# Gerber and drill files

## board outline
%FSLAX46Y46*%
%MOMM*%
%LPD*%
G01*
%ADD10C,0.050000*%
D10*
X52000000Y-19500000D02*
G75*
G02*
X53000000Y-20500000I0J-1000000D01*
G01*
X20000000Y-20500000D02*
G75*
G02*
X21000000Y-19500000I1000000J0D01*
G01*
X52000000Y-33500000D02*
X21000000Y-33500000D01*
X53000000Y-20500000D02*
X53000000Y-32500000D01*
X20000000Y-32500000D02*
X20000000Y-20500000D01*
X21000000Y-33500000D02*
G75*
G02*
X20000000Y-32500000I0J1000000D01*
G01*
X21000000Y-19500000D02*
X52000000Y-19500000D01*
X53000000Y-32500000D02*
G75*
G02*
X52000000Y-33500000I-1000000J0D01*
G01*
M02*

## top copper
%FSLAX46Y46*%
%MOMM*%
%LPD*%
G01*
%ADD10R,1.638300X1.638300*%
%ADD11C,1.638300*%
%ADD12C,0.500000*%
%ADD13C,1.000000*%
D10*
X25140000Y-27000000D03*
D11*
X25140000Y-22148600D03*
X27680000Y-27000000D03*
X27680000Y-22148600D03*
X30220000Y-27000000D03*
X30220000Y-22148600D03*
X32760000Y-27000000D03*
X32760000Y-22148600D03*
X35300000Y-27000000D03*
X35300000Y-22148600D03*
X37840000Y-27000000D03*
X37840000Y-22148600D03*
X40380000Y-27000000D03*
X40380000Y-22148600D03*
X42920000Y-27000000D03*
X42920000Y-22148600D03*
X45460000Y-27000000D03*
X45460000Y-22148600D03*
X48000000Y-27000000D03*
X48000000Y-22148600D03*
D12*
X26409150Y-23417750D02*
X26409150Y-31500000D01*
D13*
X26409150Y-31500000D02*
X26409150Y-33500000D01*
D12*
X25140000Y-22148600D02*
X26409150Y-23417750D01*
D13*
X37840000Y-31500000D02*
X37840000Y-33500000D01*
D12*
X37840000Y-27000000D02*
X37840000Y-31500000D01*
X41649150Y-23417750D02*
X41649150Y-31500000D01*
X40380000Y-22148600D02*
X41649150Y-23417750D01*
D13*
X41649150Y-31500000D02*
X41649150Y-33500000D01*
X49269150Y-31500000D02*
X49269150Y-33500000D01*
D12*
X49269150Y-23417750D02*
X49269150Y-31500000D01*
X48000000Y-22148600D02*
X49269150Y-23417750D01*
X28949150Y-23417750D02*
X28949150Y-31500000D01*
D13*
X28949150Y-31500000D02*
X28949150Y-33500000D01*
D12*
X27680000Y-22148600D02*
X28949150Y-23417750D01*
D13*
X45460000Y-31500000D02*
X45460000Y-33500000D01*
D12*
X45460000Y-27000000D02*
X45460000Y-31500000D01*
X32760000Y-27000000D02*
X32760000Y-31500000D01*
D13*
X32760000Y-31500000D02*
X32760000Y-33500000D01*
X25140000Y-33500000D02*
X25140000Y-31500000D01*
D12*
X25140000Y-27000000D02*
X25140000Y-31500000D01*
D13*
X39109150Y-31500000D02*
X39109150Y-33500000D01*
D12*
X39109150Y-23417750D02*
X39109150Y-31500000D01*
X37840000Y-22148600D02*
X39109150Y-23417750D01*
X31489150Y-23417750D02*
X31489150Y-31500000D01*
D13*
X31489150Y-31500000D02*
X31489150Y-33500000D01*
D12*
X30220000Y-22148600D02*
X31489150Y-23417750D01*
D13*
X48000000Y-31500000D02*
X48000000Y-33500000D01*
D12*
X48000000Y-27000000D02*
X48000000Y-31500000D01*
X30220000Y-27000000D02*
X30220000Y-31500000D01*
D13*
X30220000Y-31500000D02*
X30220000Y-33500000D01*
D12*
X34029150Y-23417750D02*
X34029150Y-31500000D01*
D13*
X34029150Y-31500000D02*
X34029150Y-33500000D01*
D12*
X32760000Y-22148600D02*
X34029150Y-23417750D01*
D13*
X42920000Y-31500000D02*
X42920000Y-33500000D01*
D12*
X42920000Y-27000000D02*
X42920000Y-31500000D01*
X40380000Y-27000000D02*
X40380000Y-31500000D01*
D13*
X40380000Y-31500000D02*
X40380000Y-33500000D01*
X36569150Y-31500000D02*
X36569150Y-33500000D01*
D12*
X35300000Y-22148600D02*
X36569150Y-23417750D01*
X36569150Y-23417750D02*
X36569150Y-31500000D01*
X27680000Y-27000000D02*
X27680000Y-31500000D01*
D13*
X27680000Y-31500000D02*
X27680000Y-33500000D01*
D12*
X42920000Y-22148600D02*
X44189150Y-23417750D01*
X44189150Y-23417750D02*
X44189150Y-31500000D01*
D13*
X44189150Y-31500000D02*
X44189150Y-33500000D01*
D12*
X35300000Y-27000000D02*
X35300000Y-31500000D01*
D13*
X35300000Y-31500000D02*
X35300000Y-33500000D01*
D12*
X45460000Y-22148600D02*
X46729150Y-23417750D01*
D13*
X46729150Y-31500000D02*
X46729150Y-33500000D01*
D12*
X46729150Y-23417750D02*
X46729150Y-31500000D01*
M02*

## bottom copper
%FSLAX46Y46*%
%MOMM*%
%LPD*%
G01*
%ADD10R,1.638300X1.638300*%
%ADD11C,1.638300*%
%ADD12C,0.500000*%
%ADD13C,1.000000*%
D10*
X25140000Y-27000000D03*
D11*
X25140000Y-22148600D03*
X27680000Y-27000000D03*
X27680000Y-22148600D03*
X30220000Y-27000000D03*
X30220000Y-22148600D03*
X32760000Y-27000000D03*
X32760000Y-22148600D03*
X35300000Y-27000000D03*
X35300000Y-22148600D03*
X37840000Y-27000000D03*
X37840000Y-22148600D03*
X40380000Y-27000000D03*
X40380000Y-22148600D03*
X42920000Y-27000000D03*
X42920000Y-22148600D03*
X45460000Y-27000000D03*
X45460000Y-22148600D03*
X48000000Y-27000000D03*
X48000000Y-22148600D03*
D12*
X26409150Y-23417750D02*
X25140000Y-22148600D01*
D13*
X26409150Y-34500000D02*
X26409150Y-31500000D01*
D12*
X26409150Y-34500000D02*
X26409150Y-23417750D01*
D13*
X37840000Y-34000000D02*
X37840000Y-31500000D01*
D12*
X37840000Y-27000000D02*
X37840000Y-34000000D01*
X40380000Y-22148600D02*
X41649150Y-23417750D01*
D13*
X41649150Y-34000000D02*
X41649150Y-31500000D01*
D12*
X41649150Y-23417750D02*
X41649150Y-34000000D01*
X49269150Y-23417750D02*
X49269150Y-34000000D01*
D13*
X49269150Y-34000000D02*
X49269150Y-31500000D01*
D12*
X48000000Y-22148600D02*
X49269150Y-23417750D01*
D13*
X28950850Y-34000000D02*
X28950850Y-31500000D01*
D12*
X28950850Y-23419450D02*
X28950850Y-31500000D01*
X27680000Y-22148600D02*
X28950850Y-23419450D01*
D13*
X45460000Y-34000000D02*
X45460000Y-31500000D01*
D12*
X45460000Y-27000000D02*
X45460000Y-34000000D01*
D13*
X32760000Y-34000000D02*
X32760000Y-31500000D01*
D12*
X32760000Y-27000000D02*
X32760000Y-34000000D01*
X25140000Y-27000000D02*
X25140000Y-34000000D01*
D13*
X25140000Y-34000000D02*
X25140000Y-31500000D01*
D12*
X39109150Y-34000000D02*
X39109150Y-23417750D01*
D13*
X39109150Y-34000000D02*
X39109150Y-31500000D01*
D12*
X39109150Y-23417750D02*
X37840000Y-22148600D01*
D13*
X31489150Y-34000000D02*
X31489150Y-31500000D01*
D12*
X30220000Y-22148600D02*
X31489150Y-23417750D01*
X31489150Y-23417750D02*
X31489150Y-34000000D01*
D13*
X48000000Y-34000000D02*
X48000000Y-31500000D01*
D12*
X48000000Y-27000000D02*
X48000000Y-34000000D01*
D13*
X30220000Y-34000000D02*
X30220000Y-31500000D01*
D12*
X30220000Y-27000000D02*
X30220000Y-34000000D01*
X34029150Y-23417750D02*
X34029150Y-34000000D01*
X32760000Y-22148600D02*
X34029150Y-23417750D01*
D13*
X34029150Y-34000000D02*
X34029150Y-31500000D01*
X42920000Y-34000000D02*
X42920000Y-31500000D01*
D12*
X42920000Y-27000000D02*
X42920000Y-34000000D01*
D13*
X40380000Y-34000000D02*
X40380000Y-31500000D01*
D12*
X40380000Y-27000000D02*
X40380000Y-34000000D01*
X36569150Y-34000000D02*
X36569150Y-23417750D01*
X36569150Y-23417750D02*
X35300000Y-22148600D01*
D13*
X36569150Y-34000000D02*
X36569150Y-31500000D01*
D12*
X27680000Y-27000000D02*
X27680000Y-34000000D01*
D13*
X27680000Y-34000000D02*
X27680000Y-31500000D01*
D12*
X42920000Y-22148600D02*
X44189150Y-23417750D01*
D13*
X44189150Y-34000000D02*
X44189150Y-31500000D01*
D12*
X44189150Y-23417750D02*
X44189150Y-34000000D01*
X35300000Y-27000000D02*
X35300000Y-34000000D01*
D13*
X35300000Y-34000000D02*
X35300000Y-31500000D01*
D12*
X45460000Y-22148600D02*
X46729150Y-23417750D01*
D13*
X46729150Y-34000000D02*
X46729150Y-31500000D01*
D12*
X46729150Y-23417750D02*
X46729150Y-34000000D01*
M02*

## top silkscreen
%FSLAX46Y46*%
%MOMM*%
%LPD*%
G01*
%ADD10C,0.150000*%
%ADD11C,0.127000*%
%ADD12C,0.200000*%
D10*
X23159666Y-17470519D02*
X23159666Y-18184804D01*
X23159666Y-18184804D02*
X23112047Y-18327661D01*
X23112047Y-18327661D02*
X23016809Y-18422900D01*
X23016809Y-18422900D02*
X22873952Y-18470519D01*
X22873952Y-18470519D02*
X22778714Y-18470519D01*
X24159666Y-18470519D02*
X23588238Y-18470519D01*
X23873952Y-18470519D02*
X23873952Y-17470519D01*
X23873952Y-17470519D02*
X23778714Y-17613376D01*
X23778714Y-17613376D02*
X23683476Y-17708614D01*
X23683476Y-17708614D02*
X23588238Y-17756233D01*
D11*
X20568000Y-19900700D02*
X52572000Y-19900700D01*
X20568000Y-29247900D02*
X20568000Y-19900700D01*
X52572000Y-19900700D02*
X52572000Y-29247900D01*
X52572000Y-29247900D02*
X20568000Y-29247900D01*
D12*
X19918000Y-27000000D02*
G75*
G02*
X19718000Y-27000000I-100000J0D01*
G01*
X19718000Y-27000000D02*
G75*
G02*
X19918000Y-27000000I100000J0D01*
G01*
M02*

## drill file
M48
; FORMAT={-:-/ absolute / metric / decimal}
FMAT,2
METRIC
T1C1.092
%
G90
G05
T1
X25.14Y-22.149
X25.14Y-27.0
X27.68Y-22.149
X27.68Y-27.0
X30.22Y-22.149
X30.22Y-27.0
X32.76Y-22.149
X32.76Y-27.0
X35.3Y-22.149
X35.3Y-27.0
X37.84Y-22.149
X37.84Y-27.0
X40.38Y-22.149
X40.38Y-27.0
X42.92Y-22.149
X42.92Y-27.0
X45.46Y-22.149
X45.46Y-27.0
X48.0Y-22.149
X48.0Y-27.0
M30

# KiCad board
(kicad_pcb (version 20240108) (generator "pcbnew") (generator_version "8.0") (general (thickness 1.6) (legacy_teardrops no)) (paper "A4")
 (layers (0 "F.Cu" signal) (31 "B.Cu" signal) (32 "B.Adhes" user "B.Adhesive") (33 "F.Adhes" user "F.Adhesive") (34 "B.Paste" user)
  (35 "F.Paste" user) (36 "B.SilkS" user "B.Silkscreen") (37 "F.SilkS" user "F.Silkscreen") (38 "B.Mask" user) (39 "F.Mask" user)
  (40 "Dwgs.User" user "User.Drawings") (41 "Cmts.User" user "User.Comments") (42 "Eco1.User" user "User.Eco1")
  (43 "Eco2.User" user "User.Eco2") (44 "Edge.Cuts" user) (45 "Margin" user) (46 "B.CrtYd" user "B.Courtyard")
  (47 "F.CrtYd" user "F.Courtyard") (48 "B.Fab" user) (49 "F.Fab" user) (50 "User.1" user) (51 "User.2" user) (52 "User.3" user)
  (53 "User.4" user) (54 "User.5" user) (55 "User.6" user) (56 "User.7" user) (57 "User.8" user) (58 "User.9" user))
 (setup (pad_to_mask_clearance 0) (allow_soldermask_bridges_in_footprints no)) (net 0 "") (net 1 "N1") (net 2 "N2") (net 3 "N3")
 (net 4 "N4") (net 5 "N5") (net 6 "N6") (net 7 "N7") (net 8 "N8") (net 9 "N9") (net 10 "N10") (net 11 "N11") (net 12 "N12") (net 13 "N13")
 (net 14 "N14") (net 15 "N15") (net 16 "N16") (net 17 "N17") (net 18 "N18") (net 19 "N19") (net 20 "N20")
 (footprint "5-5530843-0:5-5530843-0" (layer "F.Cu") (at 36.57 24.5743)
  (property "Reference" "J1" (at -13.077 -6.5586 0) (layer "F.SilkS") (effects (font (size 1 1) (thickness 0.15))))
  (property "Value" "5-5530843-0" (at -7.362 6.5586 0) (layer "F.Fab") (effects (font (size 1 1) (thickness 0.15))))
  (fp_line (start -16.002 -4.6736) (end 16.002 -4.6736) (stroke (width 0.127) (type solid)) (layer "F.SilkS"))
  (fp_line (start -16.002 4.6736) (end -16.002 -4.6736) (stroke (width 0.127) (type solid)) (layer "F.SilkS"))
  (fp_line (start 16.002 -4.6736) (end 16.002 4.6736) (stroke (width 0.127) (type solid)) (layer "F.SilkS"))
  (fp_line (start 16.002 4.6736) (end -16.002 4.6736) (stroke (width 0.127) (type solid)) (layer "F.SilkS"))
  (fp_circle (center -16.752 2.4257) (end -16.652 2.4257) (stroke (width 0.2) (type solid)) (fill none) (layer "F.SilkS"))
  (pad "1" thru_hole rect (at -11.43 2.4257) (size 1.6383 1.6383) (drill 1.0922) (layers "*.Cu" "*.Mask") (remove_unused_layers no)
   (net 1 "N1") (solder_mask_margin 0.102))
  (pad "2" thru_hole circle (at -11.43 -2.4257) (size 1.6383 1.6383) (drill 1.0922) (layers "*.Cu" "*.Mask") (remove_unused_layers no)
   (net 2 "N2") (solder_mask_margin 0.102))
  (pad "3" thru_hole circle (at -8.89 2.4257) (size 1.6383 1.6383) (drill 1.0922) (layers "*.Cu" "*.Mask") (remove_unused_layers no)
   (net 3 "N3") (solder_mask_margin 0.102))
  (pad "4" thru_hole circle (at -8.89 -2.4257) (size 1.6383 1.6383) (drill 1.0922) (layers "*.Cu" "*.Mask") (remove_unused_layers no)
   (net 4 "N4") (solder_mask_margin 0.102))
  (pad "5" thru_hole circle (at -6.35 2.4257) (size 1.6383 1.6383) (drill 1.0922) (layers "*.Cu" "*.Mask") (remove_unused_layers no)
   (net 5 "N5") (solder_mask_margin 0.102))
  (pad "6" thru_hole circle (at -6.35 -2.4257) (size 1.6383 1.6383) (drill 1.0922) (layers "*.Cu" "*.Mask") (remove_unused_layers no)
   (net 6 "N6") (solder_mask_margin 0.102))
  (pad "7" thru_hole circle (at -3.81 2.4257) (size 1.6383 1.6383) (drill 1.0922) (layers "*.Cu" "*.Mask") (remove_unused_layers no)
   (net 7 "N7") (solder_mask_margin 0.102))
  (pad "8" thru_hole circle (at -3.81 -2.4257) (size 1.6383 1.6383) (drill 1.0922) (layers "*.Cu" "*.Mask") (remove_unused_layers no)
   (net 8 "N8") (solder_mask_margin 0.102))
  (pad "9" thru_hole circle (at -1.27 2.4257) (size 1.6383 1.6383) (drill 1.0922) (layers "*.Cu" "*.Mask") (remove_unused_layers no)
   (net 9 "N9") (solder_mask_margin 0.102))
  (pad "10" thru_hole circle (at -1.27 -2.4257) (size 1.6383 1.6383) (drill 1.0922) (layers "*.Cu" "*.Mask") (remove_unused_layers no)
   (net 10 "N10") (solder_mask_margin 0.102))
  (pad "11" thru_hole circle (at 1.27 2.4257) (size 1.6383 1.6383) (drill 1.0922) (layers "*.Cu" "*.Mask") (remove_unused_layers no)
   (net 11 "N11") (solder_mask_margin 0.102))
  (pad "12" thru_hole circle (at 1.27 -2.4257) (size 1.6383 1.6383) (drill 1.0922) (layers "*.Cu" "*.Mask") (remove_unused_layers no)
   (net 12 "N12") (solder_mask_margin 0.102))
  (pad "13" thru_hole circle (at 3.81 2.4257) (size 1.6383 1.6383) (drill 1.0922) (layers "*.Cu" "*.Mask") (remove_unused_layers no)
   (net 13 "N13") (solder_mask_margin 0.102))
  (pad "14" thru_hole circle (at 3.81 -2.4257) (size 1.6383 1.6383) (drill 1.0922) (layers "*.Cu" "*.Mask") (remove_unused_layers no)
   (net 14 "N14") (solder_mask_margin 0.102))
  (pad "15" thru_hole circle (at 6.35 2.4257) (size 1.6383 1.6383) (drill 1.0922) (layers "*.Cu" "*.Mask") (remove_unused_layers no)
   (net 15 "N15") (solder_mask_margin 0.102))
  (pad "16" thru_hole circle (at 6.35 -2.4257) (size 1.6383 1.6383) (drill 1.0922) (layers "*.Cu" "*.Mask") (remove_unused_layers no)
   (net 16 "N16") (solder_mask_margin 0.102))
  (pad "17" thru_hole circle (at 8.89 2.4257) (size 1.6383 1.6383) (drill 1.0922) (layers "*.Cu" "*.Mask") (remove_unused_layers no)
   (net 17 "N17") (solder_mask_margin 0.102))
  (pad "18" thru_hole circle (at 8.89 -2.4257) (size 1.6383 1.6383) (drill 1.0922) (layers "*.Cu" "*.Mask") (remove_unused_layers no)
   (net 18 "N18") (solder_mask_margin 0.102))
  (pad "19" thru_hole circle (at 11.43 2.4257) (size 1.6383 1.6383) (drill 1.0922) (layers "*.Cu" "*.Mask") (remove_unused_layers no)
   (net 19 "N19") (solder_mask_margin 0.102))
  (pad "20" thru_hole circle (at 11.43 -2.4257) (size 1.6383 1.6383) (drill 1.0922) (layers "*.Cu" "*.Mask") (remove_unused_layers no)
   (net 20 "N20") (solder_mask_margin 0.102)))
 (gr_arc (start 52 19.5) (mid 52.707107 19.792893) (end 53 20.5) (stroke (width 0.05) (type default)) (layer "Edge.Cuts"))
 (gr_arc (start 20 20.5) (mid 20.292893 19.792893) (end 21 19.5) (stroke (width 0.05) (type default)) (layer "Edge.Cuts"))
 (gr_line (start 52 33.5) (end 21 33.5) (stroke (width 0.05) (type default)) (layer "Edge.Cuts"))
 (gr_line (start 53 20.5) (end 53 32.5) (stroke (width 0.05) (type default)) (layer "Edge.Cuts"))
 (gr_line (start 20 32.5) (end 20 20.5) (stroke (width 0.05) (type default)) (layer "Edge.Cuts"))
 (gr_arc (start 21 33.5) (mid 20.292893 33.207107) (end 20 32.5) (stroke (width 0.05) (type default)) (layer "Edge.Cuts"))
 (gr_line (start 21 19.5) (end 52 19.5) (stroke (width 0.05) (type default)) (layer "Edge.Cuts"))
 (gr_arc (start 53 32.5) (mid 52.707107 33.207107) (end 52 33.5) (stroke (width 0.05) (type default)) (layer "Edge.Cuts"))
 (segment (start 26.40915 23.41775) (end 26.40915 31.5) (width 0.5) (layer "F.Cu") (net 2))
 (segment (start 26.40915 31.5) (end 26.40915 33.5) (width 1) (layer "F.Cu") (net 2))
 (segment (start 25.14 22.1486) (end 26.40915 23.41775) (width 0.5) (layer "F.Cu") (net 2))
 (segment (start 26.40915 23.41775) (end 25.14 22.1486) (width 0.5) (layer "B.Cu") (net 2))
 (segment (start 26.40915 34.5) (end 26.40915 31.5) (width 1) (layer "B.Cu") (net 2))
 (segment (start 26.40915 34.5) (end 26.40915 23.41775) (width 0.5) (layer "B.Cu") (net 2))
 (segment (start 37.84 31.5) (end 37.84 33.5) (width 1) (layer "F.Cu") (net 11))
 (segment (start 37.84 27) (end 37.84 31.5) (width 0.5) (layer "F.Cu") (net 11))
 (segment (start 37.84 34) (end 37.84 31.5) (width 1) (layer "B.Cu") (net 11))
 (segment (start 37.84 27) (end 37.84 34) (width 0.5) (layer "B.Cu") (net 11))
 (segment (start 41.64915 23.41775) (end 41.64915 31.5) (width 0.5) (layer "F.Cu") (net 14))
 (segment (start 40.38 22.1486) (end 41.64915 23.41775) (width 0.5) (layer "F.Cu") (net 14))
 (segment (start 41.64915 31.5) (end 41.64915 33.5) (width 1) (layer "F.Cu") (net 14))
 (segment (start 40.38 22.1486) (end 41.64915 23.41775) (width 0.5) (layer "B.Cu") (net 14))
 (segment (start 41.64915 34) (end 41.64915 31.5) (width 1) (layer "B.Cu") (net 14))
 (segment (start 41.64915 23.41775) (end 41.64915 34) (width 0.5) (layer "B.Cu") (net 14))
 (segment (start 49.26915 31.5) (end 49.26915 33.5) (width 1) (layer "F.Cu") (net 20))
 (segment (start 49.26915 23.41775) (end 49.26915 31.5) (width 0.5) (layer "F.Cu") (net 20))
 (segment (start 48 22.1486) (end 49.26915 23.41775) (width 0.5) (layer "F.Cu") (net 20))
 (segment (start 49.26915 23.41775) (end 49.26915 34) (width 0.5) (layer "B.Cu") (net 20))
 (segment (start 49.26915 34) (end 49.26915 31.5) (width 1) (layer "B.Cu") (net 20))
 (segment (start 48 22.1486) (end 49.26915 23.41775) (width 0.5) (layer "B.Cu") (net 20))
 (segment (start 28.94915 23.41775) (end 28.94915 31.5) (width 0.5) (layer "F.Cu") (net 4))
 (segment (start 28.94915 31.5) (end 28.94915 33.5) (width 1) (layer "F.Cu") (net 4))
 (segment (start 27.68 22.1486) (end 28.94915 23.41775) (width 0.5) (layer "F.Cu") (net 4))
 (segment (start 28.95085 34) (end 28.95085 31.5) (width 1) (layer "B.Cu") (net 4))
 (segment (start 28.95085 23.41945) (end 28.95085 31.5) (width 0.5) (layer "B.Cu") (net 4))
 (segment (start 27.68 22.1486) (end 28.95085 23.41945) (width 0.5) (layer "B.Cu") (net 4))
 (segment (start 45.46 31.5) (end 45.46 33.5) (width 1) (layer "F.Cu") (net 17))
 (segment (start 45.46 27) (end 45.46 31.5) (width 0.5) (layer "F.Cu") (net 17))
 (segment (start 45.46 34) (end 45.46 31.5) (width 1) (layer "B.Cu") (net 17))
 (segment (start 45.46 27) (end 45.46 34) (width 0.5) (layer "B.Cu") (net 17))
 (segment (start 32.76 27) (end 32.76 31.5) (width 0.5) (layer "F.Cu") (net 7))
 (segment (start 32.76 31.5) (end 32.76 33.5) (width 1) (layer "F.Cu") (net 7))
 (segment (start 32.76 34) (end 32.76 31.5) (width 1) (layer "B.Cu") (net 7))
 (segment (start 32.76 27) (end 32.76 34) (width 0.5) (layer "B.Cu") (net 7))
 (segment (start 25.14 33.5) (end 25.14 31.5) (width 1) (layer "F.Cu") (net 1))
 (segment (start 25.14 27) (end 25.14 31.5) (width 0.5) (layer "F.Cu") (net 1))
 (segment (start 25.14 27) (end 25.14 34) (width 0.5) (layer "B.Cu") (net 1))
 (segment (start 25.14 34) (end 25.14 31.5) (width 1) (layer "B.Cu") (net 1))
 (segment (start 39.10915 31.5) (end 39.10915 33.5) (width 1) (layer "F.Cu") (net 12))
 (segment (start 39.10915 23.41775) (end 39.10915 31.5) (width 0.5) (layer "F.Cu") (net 12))
 (segment (start 37.84 22.1486) (end 39.10915 23.41775) (width 0.5) (layer "F.Cu") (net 12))
 (segment (start 39.10915 34) (end 39.10915 23.41775) (width 0.5) (layer "B.Cu") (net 12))
 (segment (start 39.10915 34) (end 39.10915 31.5) (width 1) (layer "B.Cu") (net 12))
 (segment (start 39.10915 23.41775) (end 37.84 22.1486) (width 0.5) (layer "B.Cu") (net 12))
 (segment (start 31.48915 23.41775) (end 31.48915 31.5) (width 0.5) (layer "F.Cu") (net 6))
 (segment (start 31.48915 31.5) (end 31.48915 33.5) (width 1) (layer "F.Cu") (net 6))
 (segment (start 30.22 22.1486) (end 31.48915 23.41775) (width 0.5) (layer "F.Cu") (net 6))
 (segment (start 31.48915 34) (end 31.48915 31.5) (width 1) (layer "B.Cu") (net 6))
 (segment (start 30.22 22.1486) (end 31.48915 23.41775) (width 0.5) (layer "B.Cu") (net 6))
 (segment (start 31.48915 23.41775) (end 31.48915 34) (width 0.5) (layer "B.Cu") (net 6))
 (segment (start 48 31.5) (end 48 33.5) (width 1) (layer "F.Cu") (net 19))
 (segment (start 48 27) (end 48 31.5) (width 0.5) (layer "F.Cu") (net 19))
 (segment (start 48 34) (end 48 31.5) (width 1) (layer "B.Cu") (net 19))
 (segment (start 48 27) (end 48 34) (width 0.5) (layer "B.Cu") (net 19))
 (segment (start 30.22 27) (end 30.22 31.5) (width 0.5) (layer "F.Cu") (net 5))
 (segment (start 30.22 31.5) (end 30.22 33.5) (width 1) (layer "F.Cu") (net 5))
 (segment (start 30.22 34) (end 30.22 31.5) (width 1) (layer "B.Cu") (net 5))
 (segment (start 30.22 27) (end 30.22 34) (width 0.5) (layer "B.Cu") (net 5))
 (segment (start 34.02915 23.41775) (end 34.02915 31.5) (width 0.5) (layer "F.Cu") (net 8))
 (segment (start 34.02915 31.5) (end 34.02915 33.5) (width 1) (layer "F.Cu") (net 8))
 (segment (start 32.76 22.1486) (end 34.02915 23.41775) (width 0.5) (layer "F.Cu") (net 8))
 (segment (start 34.02915 23.41775) (end 34.02915 34) (width 0.5) (layer "B.Cu") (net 8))
 (segment (start 32.76 22.1486) (end 34.02915 23.41775) (width 0.5) (layer "B.Cu") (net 8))
 (segment (start 34.02915 34) (end 34.02915 31.5) (width 1) (layer "B.Cu") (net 8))
 (segment (start 42.92 31.5) (end 42.92 33.5) (width 1) (layer "F.Cu") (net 15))
 (segment (start 42.92 27) (end 42.92 31.5) (width 0.5) (layer "F.Cu") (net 15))
 (segment (start 42.92 34) (end 42.92 31.5) (width 1) (layer "B.Cu") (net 15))
 (segment (start 42.92 27) (end 42.92 34) (width 0.5) (layer "B.Cu") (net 15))
 (segment (start 40.38 27) (end 40.38 31.5) (width 0.5) (layer "F.Cu") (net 13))
 (segment (start 40.38 31.5) (end 40.38 33.5) (width 1) (layer "F.Cu") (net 13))
 (segment (start 40.38 34) (end 40.38 31.5) (width 1) (layer "B.Cu") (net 13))
 (segment (start 40.38 27) (end 40.38 34) (width 0.5) (layer "B.Cu") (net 13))
 (segment (start 36.56915 31.5) (end 36.56915 33.5) (width 1) (layer "F.Cu") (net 10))
 (segment (start 35.3 22.1486) (end 36.56915 23.41775) (width 0.5) (layer "F.Cu") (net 10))
 (segment (start 36.56915 23.41775) (end 36.56915 31.5) (width 0.5) (layer "F.Cu") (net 10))
 (segment (start 36.56915 34) (end 36.56915 23.41775) (width 0.5) (layer "B.Cu") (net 10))
 (segment (start 36.56915 23.41775) (end 35.3 22.1486) (width 0.5) (layer "B.Cu") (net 10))
 (segment (start 36.56915 34) (end 36.56915 31.5) (width 1) (layer "B.Cu") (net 10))
 (segment (start 27.68 27) (end 27.68 31.5) (width 0.5) (layer "F.Cu") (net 3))
 (segment (start 27.68 31.5) (end 27.68 33.5) (width 1) (layer "F.Cu") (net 3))
 (segment (start 27.68 27) (end 27.68 34) (width 0.5) (layer "B.Cu") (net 3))
 (segment (start 27.68 34) (end 27.68 31.5) (width 1) (layer "B.Cu") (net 3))
 (segment (start 42.92 22.1486) (end 44.18915 23.41775) (width 0.5) (layer "F.Cu") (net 16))
 (segment (start 44.18915 23.41775) (end 44.18915 31.5) (width 0.5) (layer "F.Cu") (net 16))
 (segment (start 44.18915 31.5) (end 44.18915 33.5) (width 1) (layer "F.Cu") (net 16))
 (segment (start 42.92 22.1486) (end 44.18915 23.41775) (width 0.5) (layer "B.Cu") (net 16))
 (segment (start 44.18915 34) (end 44.18915 31.5) (width 1) (layer "B.Cu") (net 16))
 (segment (start 44.18915 23.41775) (end 44.18915 34) (width 0.5) (layer "B.Cu") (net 16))
 (segment (start 35.3 27) (end 35.3 31.5) (width 0.5) (layer "F.Cu") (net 9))
 (segment (start 35.3 31.5) (end 35.3 33.5) (width 1) (layer "F.Cu") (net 9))
 (segment (start 35.3 27) (end 35.3 34) (width 0.5) (layer "B.Cu") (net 9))
 (segment (start 35.3 34) (end 35.3 31.5) (width 1) (layer "B.Cu") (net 9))
 (segment (start 45.46 22.1486) (end 46.72915 23.41775) (width 0.5) (layer "F.Cu") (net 18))
 (segment (start 46.72915 31.5) (end 46.72915 33.5) (width 1) (layer "F.Cu") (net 18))
 (segment (start 46.72915 23.41775) (end 46.72915 31.5) (width 0.5) (layer "F.Cu") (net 18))
 (segment (start 45.46 22.1486) (end 46.72915 23.41775) (width 0.5) (layer "B.Cu") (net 18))
 (segment (start 46.72915 34) (end 46.72915 31.5) (width 1) (layer "B.Cu") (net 18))
 (segment (start 46.72915 23.41775) (end 46.72915 34) (width 0.5) (layer "B.Cu") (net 18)))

